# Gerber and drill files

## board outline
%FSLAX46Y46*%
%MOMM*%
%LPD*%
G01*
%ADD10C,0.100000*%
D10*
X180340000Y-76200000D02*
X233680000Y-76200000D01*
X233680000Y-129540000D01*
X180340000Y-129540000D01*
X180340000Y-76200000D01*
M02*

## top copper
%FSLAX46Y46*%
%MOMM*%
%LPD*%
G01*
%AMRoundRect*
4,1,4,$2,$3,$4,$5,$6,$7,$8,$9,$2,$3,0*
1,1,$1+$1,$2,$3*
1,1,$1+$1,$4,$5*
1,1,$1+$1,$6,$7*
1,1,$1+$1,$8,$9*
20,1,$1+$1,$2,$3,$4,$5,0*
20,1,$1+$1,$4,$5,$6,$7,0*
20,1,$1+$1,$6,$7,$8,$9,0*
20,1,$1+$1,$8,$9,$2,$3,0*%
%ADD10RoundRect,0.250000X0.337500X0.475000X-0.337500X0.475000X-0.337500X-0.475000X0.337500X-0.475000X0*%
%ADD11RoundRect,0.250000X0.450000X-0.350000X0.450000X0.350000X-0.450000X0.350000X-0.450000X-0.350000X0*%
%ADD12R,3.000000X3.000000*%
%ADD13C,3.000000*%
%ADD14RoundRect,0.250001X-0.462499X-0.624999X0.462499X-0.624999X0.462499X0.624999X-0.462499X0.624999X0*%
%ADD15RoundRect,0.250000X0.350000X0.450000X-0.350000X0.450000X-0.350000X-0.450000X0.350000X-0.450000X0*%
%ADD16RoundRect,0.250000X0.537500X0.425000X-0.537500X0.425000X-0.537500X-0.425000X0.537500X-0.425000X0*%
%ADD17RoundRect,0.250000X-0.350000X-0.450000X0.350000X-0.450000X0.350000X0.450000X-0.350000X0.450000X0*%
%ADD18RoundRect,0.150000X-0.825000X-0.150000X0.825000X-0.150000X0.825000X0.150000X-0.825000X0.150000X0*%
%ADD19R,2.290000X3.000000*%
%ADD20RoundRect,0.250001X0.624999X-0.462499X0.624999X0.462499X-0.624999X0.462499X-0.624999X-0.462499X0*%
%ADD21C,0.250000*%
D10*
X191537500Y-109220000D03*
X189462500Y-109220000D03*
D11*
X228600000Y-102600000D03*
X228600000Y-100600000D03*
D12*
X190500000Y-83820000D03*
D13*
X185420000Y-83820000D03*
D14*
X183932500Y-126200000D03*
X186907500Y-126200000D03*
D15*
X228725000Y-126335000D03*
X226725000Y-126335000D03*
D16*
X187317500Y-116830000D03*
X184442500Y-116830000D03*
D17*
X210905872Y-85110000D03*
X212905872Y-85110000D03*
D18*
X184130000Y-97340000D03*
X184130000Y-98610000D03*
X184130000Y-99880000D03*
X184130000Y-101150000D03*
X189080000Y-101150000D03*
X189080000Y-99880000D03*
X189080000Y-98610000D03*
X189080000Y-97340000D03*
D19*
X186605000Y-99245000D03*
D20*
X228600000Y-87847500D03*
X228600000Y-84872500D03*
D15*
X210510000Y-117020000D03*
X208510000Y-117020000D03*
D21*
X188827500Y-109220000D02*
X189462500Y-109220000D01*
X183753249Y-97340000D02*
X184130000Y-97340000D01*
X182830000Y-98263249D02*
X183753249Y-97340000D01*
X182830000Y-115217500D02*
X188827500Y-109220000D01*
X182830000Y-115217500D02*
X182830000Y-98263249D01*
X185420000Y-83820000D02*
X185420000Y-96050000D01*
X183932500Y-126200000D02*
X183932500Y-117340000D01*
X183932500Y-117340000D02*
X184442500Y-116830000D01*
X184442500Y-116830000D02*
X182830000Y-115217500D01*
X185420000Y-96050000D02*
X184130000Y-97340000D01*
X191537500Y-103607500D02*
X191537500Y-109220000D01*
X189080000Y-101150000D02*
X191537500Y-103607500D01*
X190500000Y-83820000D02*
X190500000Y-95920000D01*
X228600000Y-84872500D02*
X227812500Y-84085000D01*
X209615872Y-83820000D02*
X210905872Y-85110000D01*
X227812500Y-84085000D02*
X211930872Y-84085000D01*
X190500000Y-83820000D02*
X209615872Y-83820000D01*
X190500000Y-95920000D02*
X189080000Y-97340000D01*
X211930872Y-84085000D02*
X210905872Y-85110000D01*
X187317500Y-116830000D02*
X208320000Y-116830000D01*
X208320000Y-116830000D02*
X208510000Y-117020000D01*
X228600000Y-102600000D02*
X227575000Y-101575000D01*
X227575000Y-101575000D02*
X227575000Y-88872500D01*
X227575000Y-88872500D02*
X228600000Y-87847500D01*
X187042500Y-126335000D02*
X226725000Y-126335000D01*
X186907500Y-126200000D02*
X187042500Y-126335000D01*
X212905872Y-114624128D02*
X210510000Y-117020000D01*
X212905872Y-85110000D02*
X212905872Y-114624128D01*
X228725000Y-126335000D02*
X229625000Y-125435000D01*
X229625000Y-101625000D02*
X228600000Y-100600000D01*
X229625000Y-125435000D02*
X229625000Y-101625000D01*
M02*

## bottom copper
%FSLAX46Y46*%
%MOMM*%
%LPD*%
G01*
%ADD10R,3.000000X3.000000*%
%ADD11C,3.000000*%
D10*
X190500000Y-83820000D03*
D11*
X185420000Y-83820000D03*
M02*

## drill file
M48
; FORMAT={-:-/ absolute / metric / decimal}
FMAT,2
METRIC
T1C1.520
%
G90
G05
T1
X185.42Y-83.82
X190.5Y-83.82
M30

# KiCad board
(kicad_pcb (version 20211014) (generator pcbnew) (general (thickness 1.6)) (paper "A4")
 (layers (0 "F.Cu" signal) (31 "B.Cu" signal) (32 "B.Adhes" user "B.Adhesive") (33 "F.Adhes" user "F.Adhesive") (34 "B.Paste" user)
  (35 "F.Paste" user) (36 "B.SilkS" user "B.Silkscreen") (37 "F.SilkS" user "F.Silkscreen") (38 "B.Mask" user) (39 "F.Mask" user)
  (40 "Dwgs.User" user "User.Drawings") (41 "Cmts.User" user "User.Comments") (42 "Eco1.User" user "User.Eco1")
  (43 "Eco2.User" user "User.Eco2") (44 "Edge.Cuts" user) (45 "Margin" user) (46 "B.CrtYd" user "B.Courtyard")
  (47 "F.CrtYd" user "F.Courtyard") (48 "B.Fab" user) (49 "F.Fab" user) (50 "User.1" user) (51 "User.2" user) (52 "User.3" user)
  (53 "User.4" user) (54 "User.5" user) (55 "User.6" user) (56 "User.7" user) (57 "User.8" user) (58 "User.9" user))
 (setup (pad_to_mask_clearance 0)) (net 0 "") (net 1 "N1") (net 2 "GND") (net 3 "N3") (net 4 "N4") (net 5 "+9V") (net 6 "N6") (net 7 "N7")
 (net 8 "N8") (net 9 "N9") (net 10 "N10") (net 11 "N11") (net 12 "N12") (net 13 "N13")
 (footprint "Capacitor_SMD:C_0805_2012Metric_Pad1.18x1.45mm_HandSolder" (layer "F.Cu") (at 190.5 109.22 180)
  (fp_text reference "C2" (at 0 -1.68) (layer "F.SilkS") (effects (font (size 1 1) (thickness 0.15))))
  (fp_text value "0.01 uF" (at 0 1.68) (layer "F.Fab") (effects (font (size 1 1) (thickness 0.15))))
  (pad "1" smd roundrect (at -1.0375 0 180) (size 1.175 1.45) (layers "F.Cu" "F.Paste" "F.Mask") (roundrect_rratio 0.2127659574)
   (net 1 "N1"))
  (pad "2" smd roundrect (at 1.0375 0 180) (size 1.175 1.45) (layers "F.Cu" "F.Paste" "F.Mask") (roundrect_rratio 0.2127659574)
   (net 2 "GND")))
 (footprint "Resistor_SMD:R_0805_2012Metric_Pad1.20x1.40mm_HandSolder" (layer "F.Cu") (at 228.6 101.6 90)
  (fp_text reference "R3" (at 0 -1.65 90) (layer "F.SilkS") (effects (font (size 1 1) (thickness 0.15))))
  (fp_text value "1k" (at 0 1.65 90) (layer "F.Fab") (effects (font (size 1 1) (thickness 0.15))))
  (pad "1" smd roundrect (at -1 0 90) (size 1.2 1.4) (layers "F.Cu" "F.Paste" "F.Mask") (roundrect_rratio 0.2083333333) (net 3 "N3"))
  (pad "2" smd roundrect (at 1 0 90) (size 1.2 1.4) (layers "F.Cu" "F.Paste" "F.Mask") (roundrect_rratio 0.2083333333) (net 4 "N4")))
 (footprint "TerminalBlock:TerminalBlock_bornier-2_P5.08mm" (layer "F.Cu") (at 190.5 83.82 180)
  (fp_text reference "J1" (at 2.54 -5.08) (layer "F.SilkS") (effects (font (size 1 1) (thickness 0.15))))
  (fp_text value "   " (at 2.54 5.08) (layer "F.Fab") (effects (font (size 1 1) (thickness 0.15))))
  (pad "1" thru_hole rect (at 0 0 180) (size 3 3) (drill 1.52) (layers *.Cu *.Mask) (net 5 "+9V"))
  (pad "2" thru_hole circle (at 5.08 0 180) (size 3 3) (drill 1.52) (layers *.Cu *.Mask) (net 2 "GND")))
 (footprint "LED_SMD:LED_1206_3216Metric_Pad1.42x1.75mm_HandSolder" (layer "F.Cu") (at 185.42 126.2)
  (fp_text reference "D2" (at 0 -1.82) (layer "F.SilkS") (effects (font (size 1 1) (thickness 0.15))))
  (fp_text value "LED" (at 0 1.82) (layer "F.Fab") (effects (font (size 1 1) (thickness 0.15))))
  (pad "1" smd roundrect (at -1.4875 0) (size 1.425 1.75) (layers "F.Cu" "F.Paste" "F.Mask") (roundrect_rratio 0.1754392982) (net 2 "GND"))
  (pad "2" smd roundrect (at 1.4875 0) (size 1.425 1.75) (layers "F.Cu" "F.Paste" "F.Mask") (roundrect_rratio 0.1754392982) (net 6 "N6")))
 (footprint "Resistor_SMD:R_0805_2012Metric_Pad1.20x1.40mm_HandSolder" (layer "F.Cu") (at 227.725 126.335 180)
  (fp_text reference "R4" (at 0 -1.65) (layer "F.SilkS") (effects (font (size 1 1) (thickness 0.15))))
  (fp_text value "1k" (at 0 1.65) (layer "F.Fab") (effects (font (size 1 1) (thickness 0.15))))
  (pad "1" smd roundrect (at -1 0 180) (size 1.2 1.4) (layers "F.Cu" "F.Paste" "F.Mask") (roundrect_rratio 0.2083333333) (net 4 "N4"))
  (pad "2" smd roundrect (at 1 0 180) (size 1.2 1.4) (layers "F.Cu" "F.Paste" "F.Mask") (roundrect_rratio 0.2083333333) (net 6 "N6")))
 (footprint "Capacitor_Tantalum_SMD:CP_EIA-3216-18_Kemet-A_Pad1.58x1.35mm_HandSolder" (layer "F.Cu") (at 185.88 116.83 180)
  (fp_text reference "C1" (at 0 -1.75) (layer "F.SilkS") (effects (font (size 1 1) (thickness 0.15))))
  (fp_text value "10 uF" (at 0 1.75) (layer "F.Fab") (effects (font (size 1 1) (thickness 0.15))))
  (pad "1" smd roundrect (at -1.4375 0 180) (size 1.575 1.35) (layers "F.Cu" "F.Paste" "F.Mask") (roundrect_rratio 0.1851851852)
   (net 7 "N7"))
  (pad "2" smd roundrect (at 1.4375 0 180) (size 1.575 1.35) (layers "F.Cu" "F.Paste" "F.Mask") (roundrect_rratio 0.1851851852)
   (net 2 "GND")))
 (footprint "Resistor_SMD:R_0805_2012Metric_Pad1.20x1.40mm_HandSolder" (layer "F.Cu") (at 211.905872 85.11)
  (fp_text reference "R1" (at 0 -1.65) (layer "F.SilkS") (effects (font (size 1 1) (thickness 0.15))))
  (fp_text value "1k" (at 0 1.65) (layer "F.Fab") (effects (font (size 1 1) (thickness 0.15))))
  (pad "1" smd roundrect (at -1 0) (size 1.2 1.4) (layers "F.Cu" "F.Paste" "F.Mask") (roundrect_rratio 0.2083333333) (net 5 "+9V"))
  (pad "2" smd roundrect (at 1 0) (size 1.2 1.4) (layers "F.Cu" "F.Paste" "F.Mask") (roundrect_rratio 0.2083333333) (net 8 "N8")))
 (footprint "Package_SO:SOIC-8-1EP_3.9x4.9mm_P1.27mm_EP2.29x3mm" (layer "F.Cu") (at 186.605 99.245)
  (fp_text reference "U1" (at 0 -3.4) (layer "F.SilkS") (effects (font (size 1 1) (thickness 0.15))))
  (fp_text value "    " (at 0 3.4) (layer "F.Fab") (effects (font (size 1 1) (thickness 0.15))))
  (pad "" smd roundrect (at 0.57 -0.75) (size 0.92 1.21) (layers "F.Paste") (roundrect_rratio 0.25))
  (pad "" smd roundrect (at -0.57 0.75) (size 0.92 1.21) (layers "F.Paste") (roundrect_rratio 0.25))
  (pad "" smd roundrect (at -0.57 -0.75) (size 0.92 1.21) (layers "F.Paste") (roundrect_rratio 0.25))
  (pad "" smd roundrect (at 0.57 0.75) (size 0.92 1.21) (layers "F.Paste") (roundrect_rratio 0.25))
  (pad "1" smd roundrect (at -2.475 -1.905) (size 1.95 0.6) (layers "F.Cu" "F.Paste" "F.Mask") (roundrect_rratio 0.25) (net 2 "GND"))
  (pad "2" smd roundrect (at -2.475 -0.635) (size 1.95 0.6) (layers "F.Cu" "F.Paste" "F.Mask") (roundrect_rratio 0.25) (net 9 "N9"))
  (pad "3" smd roundrect (at -2.475 0.635) (size 1.95 0.6) (layers "F.Cu" "F.Paste" "F.Mask") (roundrect_rratio 0.25) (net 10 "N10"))
  (pad "4" smd roundrect (at -2.475 1.905) (size 1.95 0.6) (layers "F.Cu" "F.Paste" "F.Mask") (roundrect_rratio 0.25) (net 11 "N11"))
  (pad "5" smd roundrect (at 2.475 1.905) (size 1.95 0.6) (layers "F.Cu" "F.Paste" "F.Mask") (roundrect_rratio 0.25) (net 1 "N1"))
  (pad "6" smd roundrect (at 2.475 0.635) (size 1.95 0.6) (layers "F.Cu" "F.Paste" "F.Mask") (roundrect_rratio 0.25) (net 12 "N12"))
  (pad "7" smd roundrect (at 2.475 -0.635) (size 1.95 0.6) (layers "F.Cu" "F.Paste" "F.Mask") (roundrect_rratio 0.25) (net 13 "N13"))
  (pad "8" smd roundrect (at 2.475 -1.905) (size 1.95 0.6) (layers "F.Cu" "F.Paste" "F.Mask") (roundrect_rratio 0.25) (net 5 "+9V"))
  (pad "9" smd rect (at 0 0) (size 2.29 3) (layers "F.Cu" "F.Mask")))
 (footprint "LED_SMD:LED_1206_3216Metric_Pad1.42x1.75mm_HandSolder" (layer "F.Cu") (at 228.6 86.36 90)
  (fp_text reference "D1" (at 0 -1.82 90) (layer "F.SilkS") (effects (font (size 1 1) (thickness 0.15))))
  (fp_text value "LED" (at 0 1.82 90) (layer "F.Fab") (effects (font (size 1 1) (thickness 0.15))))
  (pad "1" smd roundrect (at -1.4875 0 90) (size 1.425 1.75) (layers "F.Cu" "F.Paste" "F.Mask") (roundrect_rratio 0.1754392982) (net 3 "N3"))
  (pad "2" smd roundrect (at 1.4875 0 90) (size 1.425 1.75) (layers "F.Cu" "F.Paste" "F.Mask") (roundrect_rratio 0.1754392982) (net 5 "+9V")))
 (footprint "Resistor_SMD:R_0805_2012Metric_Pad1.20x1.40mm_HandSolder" (layer "F.Cu") (at 209.51 117.02 180)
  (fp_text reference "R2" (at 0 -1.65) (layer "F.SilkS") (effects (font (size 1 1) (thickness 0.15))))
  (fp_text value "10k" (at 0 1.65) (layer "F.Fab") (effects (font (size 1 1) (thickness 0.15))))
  (pad "1" smd roundrect (at -1 0 180) (size 1.2 1.4) (layers "F.Cu" "F.Paste" "F.Mask") (roundrect_rratio 0.2083333333) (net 8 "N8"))
  (pad "2" smd roundrect (at 1 0 180) (size 1.2 1.4) (layers "F.Cu" "F.Paste" "F.Mask") (roundrect_rratio 0.2083333333) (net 7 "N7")))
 (gr_rect (start 180.34 76.2) (end 233.68 129.54) (layer "Edge.Cuts") (width 0.1) (fill none))
 (segment (start 188.8275 109.22) (end 189.4625 109.22) (width 0.25) (layer "F.Cu") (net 2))
 (segment (start 183.753249 97.34) (end 184.13 97.34) (width 0.25) (layer "F.Cu") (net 2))
 (segment (start 182.83 98.263249) (end 183.753249 97.34) (width 0.25) (layer "F.Cu") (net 2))
 (segment (start 182.83 115.2175) (end 188.8275 109.22) (width 0.25) (layer "F.Cu") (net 2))
 (segment (start 182.83 115.2175) (end 182.83 98.263249) (width 0.25) (layer "F.Cu") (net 2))
 (segment (start 185.42 83.82) (end 185.42 96.05) (width 0.25) (layer "F.Cu") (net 2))
 (segment (start 183.9325 126.2) (end 183.9325 117.34) (width 0.25) (layer "F.Cu") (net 2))
 (segment (start 183.9325 117.34) (end 184.4425 116.83) (width 0.25) (layer "F.Cu") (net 2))
 (segment (start 184.4425 116.83) (end 182.83 115.2175) (width 0.25) (layer "F.Cu") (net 2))
 (segment (start 185.42 96.05) (end 184.13 97.34) (width 0.25) (layer "F.Cu") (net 2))
 (segment (start 191.5375 103.6075) (end 191.5375 109.22) (width 0.25) (layer "F.Cu") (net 1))
 (segment (start 189.08 101.15) (end 191.5375 103.6075) (width 0.25) (layer "F.Cu") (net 1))
 (segment (start 190.5 83.82) (end 190.5 95.92) (width 0.25) (layer "F.Cu") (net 5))
 (segment (start 228.6 84.8725) (end 227.8125 84.085) (width 0.25) (layer "F.Cu") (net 5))
 (segment (start 209.615872 83.82) (end 210.905872 85.11) (width 0.25) (layer "F.Cu") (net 5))
 (segment (start 227.8125 84.085) (end 211.930872 84.085) (width 0.25) (layer "F.Cu") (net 5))
 (segment (start 190.5 83.82) (end 209.615872 83.82) (width 0.25) (layer "F.Cu") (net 5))
 (segment (start 190.5 95.92) (end 189.08 97.34) (width 0.25) (layer "F.Cu") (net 5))
 (segment (start 211.930872 84.085) (end 210.905872 85.11) (width 0.25) (layer "F.Cu") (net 5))
 (segment (start 187.3175 116.83) (end 208.32 116.83) (width 0.25) (layer "F.Cu") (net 7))
 (segment (start 208.32 116.83) (end 208.51 117.02) (width 0.25) (layer "F.Cu") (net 7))
 (segment (start 228.6 102.6) (end 227.575 101.575) (width 0.25) (layer "F.Cu") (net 3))
 (segment (start 227.575 101.575) (end 227.575 88.8725) (width 0.25) (layer "F.Cu") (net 3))
 (segment (start 227.575 88.8725) (end 228.6 87.8475) (width 0.25) (layer "F.Cu") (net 3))
 (segment (start 187.0425 126.335) (end 226.725 126.335) (width 0.25) (layer "F.Cu") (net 6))
 (segment (start 186.9075 126.2) (end 187.0425 126.335) (width 0.25) (layer "F.Cu") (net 6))
 (segment (start 212.905872 114.624128) (end 210.51 117.02) (width 0.25) (layer "F.Cu") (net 8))
 (segment (start 212.905872 85.11) (end 212.905872 114.624128) (width 0.25) (layer "F.Cu") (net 8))
 (segment (start 228.725 126.335) (end 229.625 125.435) (width 0.25) (layer "F.Cu") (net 4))
 (segment (start 229.625 101.625) (end 228.6 100.6) (width 0.25) (layer "F.Cu") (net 4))
 (segment (start 229.625 125.435) (end 229.625 101.625) (width 0.25) (layer "F.Cu") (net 4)))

